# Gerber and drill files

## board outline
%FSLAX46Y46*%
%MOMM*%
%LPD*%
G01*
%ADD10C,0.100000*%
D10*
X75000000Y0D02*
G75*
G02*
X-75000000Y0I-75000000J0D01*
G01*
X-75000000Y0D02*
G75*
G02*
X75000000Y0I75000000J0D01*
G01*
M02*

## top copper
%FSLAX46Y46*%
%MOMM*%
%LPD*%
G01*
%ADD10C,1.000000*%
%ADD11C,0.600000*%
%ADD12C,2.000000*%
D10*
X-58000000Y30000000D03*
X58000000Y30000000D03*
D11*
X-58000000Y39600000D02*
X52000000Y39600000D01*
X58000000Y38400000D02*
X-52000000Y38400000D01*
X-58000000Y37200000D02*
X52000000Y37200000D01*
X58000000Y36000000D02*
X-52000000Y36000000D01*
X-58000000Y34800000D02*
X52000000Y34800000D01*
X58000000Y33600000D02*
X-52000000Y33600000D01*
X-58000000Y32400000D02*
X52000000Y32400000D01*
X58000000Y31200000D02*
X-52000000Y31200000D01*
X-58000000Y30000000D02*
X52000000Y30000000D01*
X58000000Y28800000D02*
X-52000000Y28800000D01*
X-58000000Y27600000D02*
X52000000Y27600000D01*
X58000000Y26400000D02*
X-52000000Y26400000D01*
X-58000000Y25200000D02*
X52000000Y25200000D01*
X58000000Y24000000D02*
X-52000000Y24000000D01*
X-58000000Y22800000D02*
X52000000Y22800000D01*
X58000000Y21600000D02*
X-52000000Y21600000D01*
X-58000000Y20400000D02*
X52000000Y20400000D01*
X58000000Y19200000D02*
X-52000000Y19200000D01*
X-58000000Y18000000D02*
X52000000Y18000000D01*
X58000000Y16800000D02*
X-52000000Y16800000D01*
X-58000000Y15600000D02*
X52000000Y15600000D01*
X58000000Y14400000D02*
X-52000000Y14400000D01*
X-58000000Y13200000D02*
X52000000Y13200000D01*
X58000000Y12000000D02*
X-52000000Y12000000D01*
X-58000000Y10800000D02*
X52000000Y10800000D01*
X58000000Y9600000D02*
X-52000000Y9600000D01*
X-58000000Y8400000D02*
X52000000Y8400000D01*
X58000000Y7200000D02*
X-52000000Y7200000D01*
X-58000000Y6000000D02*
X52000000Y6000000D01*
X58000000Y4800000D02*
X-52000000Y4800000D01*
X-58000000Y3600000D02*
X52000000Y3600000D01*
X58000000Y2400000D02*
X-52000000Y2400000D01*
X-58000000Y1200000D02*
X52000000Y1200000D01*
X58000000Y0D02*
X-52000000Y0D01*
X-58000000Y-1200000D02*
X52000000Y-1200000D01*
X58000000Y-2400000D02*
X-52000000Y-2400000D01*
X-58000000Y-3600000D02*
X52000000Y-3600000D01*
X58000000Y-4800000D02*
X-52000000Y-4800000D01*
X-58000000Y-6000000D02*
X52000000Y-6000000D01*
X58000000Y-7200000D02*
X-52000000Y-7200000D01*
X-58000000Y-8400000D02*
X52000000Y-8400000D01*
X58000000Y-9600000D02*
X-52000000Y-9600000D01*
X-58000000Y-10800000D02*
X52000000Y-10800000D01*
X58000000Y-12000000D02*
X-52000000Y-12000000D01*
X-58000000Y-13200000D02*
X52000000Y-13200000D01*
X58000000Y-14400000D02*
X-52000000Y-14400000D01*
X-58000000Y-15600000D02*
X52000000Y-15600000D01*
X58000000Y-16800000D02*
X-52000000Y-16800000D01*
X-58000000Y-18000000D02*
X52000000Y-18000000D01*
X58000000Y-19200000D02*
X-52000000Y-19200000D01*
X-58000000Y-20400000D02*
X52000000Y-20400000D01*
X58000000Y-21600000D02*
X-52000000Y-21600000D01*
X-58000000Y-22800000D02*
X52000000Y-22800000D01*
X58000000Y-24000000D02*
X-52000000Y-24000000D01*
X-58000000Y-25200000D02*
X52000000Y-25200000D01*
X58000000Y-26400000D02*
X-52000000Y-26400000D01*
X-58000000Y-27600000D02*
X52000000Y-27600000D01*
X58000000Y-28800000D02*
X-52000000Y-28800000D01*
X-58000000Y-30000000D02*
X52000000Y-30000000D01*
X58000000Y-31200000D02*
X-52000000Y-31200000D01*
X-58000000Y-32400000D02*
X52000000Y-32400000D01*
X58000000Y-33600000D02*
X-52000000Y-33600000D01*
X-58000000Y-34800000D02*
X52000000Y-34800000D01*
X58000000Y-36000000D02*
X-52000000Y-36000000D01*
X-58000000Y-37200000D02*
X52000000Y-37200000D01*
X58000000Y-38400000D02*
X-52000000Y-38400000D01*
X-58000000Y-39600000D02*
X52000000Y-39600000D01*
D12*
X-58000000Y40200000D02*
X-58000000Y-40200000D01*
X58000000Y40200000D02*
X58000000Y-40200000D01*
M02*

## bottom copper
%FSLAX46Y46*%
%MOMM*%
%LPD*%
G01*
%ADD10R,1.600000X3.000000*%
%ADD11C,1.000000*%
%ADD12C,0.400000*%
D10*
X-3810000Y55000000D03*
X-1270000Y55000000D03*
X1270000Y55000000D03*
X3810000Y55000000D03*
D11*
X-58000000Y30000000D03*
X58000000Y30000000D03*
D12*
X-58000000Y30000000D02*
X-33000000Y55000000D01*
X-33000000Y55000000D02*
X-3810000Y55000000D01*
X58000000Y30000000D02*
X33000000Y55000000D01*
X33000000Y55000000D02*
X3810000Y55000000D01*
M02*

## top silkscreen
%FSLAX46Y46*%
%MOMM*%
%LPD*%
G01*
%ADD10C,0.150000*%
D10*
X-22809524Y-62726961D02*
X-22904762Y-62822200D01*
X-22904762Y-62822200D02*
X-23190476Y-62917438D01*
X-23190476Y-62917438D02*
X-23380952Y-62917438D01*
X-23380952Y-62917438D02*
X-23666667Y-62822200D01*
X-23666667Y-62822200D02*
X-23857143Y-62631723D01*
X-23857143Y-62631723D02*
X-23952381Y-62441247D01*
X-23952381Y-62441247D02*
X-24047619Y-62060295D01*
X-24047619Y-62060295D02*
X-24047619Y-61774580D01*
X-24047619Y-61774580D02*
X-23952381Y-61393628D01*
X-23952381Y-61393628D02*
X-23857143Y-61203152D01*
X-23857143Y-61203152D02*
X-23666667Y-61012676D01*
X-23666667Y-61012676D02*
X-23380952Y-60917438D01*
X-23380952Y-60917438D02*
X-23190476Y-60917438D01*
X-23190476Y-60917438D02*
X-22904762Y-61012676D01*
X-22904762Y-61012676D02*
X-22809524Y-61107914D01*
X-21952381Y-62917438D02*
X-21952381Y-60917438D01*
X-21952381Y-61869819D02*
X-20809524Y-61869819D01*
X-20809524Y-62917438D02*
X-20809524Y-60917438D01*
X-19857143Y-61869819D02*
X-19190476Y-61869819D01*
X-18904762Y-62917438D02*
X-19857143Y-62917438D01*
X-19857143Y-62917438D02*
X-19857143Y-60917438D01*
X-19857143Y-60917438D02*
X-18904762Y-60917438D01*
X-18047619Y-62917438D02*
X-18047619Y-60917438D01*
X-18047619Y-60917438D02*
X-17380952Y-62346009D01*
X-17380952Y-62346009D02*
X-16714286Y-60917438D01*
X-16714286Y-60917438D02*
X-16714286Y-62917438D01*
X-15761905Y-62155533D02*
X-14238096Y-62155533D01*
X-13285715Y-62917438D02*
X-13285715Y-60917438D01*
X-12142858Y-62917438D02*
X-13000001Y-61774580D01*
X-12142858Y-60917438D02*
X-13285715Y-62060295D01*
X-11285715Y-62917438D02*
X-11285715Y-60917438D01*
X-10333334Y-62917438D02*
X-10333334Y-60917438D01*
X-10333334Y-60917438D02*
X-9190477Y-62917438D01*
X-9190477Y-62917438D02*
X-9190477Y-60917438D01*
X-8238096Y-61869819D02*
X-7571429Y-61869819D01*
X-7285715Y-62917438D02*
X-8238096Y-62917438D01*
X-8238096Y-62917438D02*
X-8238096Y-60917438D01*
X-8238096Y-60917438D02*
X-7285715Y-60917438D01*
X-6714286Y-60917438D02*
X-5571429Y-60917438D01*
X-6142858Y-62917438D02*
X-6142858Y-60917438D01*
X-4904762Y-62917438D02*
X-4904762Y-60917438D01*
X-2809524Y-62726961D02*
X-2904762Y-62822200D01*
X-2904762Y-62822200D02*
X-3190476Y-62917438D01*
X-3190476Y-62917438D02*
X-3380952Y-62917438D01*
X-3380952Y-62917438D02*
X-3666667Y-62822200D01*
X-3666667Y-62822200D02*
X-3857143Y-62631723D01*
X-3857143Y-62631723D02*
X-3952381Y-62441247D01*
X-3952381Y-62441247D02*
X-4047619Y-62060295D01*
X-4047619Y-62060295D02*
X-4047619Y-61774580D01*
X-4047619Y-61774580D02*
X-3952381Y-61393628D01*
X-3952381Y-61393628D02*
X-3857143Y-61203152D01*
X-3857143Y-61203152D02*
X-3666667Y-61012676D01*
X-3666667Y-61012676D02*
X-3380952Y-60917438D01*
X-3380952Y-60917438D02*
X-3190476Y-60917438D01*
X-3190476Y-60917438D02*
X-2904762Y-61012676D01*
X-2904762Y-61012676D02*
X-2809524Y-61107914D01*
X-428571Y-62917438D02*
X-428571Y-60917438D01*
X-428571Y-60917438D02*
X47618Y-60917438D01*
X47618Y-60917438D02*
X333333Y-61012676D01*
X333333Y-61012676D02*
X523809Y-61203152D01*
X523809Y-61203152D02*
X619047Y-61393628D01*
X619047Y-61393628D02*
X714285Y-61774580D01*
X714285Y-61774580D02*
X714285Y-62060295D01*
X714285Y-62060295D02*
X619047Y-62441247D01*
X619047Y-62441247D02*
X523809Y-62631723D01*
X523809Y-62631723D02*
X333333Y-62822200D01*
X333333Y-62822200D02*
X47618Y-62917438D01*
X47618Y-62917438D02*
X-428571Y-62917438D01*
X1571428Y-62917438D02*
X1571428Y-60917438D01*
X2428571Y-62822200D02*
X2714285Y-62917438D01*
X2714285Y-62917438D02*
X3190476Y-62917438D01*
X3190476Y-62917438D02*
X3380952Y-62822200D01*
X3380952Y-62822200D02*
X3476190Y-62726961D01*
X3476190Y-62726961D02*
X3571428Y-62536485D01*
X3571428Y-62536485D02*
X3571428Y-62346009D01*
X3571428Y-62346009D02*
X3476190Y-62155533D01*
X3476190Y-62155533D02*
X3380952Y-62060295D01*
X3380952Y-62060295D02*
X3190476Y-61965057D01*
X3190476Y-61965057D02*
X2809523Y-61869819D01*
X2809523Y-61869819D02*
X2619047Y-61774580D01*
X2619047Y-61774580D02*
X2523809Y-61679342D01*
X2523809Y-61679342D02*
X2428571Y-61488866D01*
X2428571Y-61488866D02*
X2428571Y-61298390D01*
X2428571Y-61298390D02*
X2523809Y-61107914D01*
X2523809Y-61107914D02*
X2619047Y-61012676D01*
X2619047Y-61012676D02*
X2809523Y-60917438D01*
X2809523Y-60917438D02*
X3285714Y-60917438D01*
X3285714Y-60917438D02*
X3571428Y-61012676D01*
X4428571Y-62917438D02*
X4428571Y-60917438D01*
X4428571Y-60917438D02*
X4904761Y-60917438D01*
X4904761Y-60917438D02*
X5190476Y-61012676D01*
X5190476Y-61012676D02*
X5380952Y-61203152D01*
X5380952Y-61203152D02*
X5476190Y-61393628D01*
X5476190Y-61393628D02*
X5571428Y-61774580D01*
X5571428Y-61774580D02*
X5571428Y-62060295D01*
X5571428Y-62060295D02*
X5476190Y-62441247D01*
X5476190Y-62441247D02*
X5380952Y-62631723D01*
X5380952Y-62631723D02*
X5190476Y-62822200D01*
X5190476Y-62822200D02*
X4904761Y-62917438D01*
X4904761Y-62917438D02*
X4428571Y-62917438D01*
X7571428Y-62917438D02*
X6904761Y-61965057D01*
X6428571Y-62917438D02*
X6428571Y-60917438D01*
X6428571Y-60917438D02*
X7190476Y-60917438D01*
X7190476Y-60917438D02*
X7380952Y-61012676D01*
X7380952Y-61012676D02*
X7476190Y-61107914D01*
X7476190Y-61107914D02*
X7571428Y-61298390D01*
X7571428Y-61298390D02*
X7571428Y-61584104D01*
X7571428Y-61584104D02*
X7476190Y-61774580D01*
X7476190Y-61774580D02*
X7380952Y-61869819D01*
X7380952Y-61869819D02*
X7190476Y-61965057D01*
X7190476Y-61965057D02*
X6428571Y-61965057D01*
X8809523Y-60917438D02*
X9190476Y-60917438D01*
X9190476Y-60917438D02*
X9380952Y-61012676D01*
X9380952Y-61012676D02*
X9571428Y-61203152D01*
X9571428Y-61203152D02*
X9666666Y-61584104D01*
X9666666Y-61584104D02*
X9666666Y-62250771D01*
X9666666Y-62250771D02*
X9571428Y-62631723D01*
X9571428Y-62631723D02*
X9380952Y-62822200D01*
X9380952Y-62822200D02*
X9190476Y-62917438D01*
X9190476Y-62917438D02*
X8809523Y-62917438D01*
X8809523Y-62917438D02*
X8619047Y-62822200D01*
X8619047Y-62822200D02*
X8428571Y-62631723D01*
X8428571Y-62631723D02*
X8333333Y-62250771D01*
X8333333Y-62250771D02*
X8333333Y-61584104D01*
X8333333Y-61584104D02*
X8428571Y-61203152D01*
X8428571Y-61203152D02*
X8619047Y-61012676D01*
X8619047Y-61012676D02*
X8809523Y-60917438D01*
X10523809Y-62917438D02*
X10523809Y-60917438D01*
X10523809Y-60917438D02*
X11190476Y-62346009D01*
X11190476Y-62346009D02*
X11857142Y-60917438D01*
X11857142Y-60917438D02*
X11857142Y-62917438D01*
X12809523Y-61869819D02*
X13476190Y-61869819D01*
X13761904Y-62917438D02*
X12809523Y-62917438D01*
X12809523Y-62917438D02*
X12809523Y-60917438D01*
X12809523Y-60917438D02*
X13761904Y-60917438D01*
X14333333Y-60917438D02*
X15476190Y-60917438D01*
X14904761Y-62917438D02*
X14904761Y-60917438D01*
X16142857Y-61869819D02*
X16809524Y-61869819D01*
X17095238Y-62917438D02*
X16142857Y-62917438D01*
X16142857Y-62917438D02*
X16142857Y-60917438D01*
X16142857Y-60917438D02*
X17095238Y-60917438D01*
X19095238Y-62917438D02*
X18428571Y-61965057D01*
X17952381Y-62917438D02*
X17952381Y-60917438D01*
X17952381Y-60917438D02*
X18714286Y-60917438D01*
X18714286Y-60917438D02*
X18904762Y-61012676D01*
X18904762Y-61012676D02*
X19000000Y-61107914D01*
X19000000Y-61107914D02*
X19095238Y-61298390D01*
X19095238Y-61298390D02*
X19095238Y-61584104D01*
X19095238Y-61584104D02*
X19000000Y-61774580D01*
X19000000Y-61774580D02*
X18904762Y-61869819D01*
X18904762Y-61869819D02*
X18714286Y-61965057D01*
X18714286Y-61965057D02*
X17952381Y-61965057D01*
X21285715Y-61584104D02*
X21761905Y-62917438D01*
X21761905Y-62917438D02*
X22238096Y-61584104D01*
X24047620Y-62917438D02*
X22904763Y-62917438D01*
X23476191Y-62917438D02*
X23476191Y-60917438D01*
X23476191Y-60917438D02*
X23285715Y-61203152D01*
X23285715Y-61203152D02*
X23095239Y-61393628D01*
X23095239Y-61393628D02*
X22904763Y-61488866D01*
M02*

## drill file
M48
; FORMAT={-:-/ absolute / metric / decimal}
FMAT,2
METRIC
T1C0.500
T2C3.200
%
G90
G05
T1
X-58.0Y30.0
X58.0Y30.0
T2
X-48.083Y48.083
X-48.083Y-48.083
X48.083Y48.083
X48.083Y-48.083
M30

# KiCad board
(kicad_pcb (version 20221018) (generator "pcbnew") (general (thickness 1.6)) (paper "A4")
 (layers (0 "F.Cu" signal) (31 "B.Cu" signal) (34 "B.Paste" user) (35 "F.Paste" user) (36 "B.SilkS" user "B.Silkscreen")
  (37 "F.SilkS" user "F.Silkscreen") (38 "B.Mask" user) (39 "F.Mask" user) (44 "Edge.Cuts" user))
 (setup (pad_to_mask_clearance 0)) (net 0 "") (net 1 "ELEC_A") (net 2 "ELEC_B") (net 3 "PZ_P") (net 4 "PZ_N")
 (segment (start -58.000 -39.600) (end 52.000 -39.600) (width 0.6) (layer "F.Cu") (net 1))
 (segment (start 58.000 -38.400) (end -52.000 -38.400) (width 0.6) (layer "F.Cu") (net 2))
 (segment (start -58.000 -37.200) (end 52.000 -37.200) (width 0.6) (layer "F.Cu") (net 1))
 (segment (start 58.000 -36.000) (end -52.000 -36.000) (width 0.6) (layer "F.Cu") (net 2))
 (segment (start -58.000 -34.800) (end 52.000 -34.800) (width 0.6) (layer "F.Cu") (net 1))
 (segment (start 58.000 -33.600) (end -52.000 -33.600) (width 0.6) (layer "F.Cu") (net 2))
 (segment (start -58.000 -32.400) (end 52.000 -32.400) (width 0.6) (layer "F.Cu") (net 1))
 (segment (start 58.000 -31.200) (end -52.000 -31.200) (width 0.6) (layer "F.Cu") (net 2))
 (segment (start -58.000 -30.000) (end 52.000 -30.000) (width 0.6) (layer "F.Cu") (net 1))
 (segment (start 58.000 -28.800) (end -52.000 -28.800) (width 0.6) (layer "F.Cu") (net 2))
 (segment (start -58.000 -27.600) (end 52.000 -27.600) (width 0.6) (layer "F.Cu") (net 1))
 (segment (start 58.000 -26.400) (end -52.000 -26.400) (width 0.6) (layer "F.Cu") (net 2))
 (segment (start -58.000 -25.200) (end 52.000 -25.200) (width 0.6) (layer "F.Cu") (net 1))
 (segment (start 58.000 -24.000) (end -52.000 -24.000) (width 0.6) (layer "F.Cu") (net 2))
 (segment (start -58.000 -22.800) (end 52.000 -22.800) (width 0.6) (layer "F.Cu") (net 1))
 (segment (start 58.000 -21.600) (end -52.000 -21.600) (width 0.6) (layer "F.Cu") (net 2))
 (segment (start -58.000 -20.400) (end 52.000 -20.400) (width 0.6) (layer "F.Cu") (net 1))
 (segment (start 58.000 -19.200) (end -52.000 -19.200) (width 0.6) (layer "F.Cu") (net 2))
 (segment (start -58.000 -18.000) (end 52.000 -18.000) (width 0.6) (layer "F.Cu") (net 1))
 (segment (start 58.000 -16.800) (end -52.000 -16.800) (width 0.6) (layer "F.Cu") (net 2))
 (segment (start -58.000 -15.600) (end 52.000 -15.600) (width 0.6) (layer "F.Cu") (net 1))
 (segment (start 58.000 -14.400) (end -52.000 -14.400) (width 0.6) (layer "F.Cu") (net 2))
 (segment (start -58.000 -13.200) (end 52.000 -13.200) (width 0.6) (layer "F.Cu") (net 1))
 (segment (start 58.000 -12.000) (end -52.000 -12.000) (width 0.6) (layer "F.Cu") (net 2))
 (segment (start -58.000 -10.800) (end 52.000 -10.800) (width 0.6) (layer "F.Cu") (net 1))
 (segment (start 58.000 -9.600) (end -52.000 -9.600) (width 0.6) (layer "F.Cu") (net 2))
 (segment (start -58.000 -8.400) (end 52.000 -8.400) (width 0.6) (layer "F.Cu") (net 1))
 (segment (start 58.000 -7.200) (end -52.000 -7.200) (width 0.6) (layer "F.Cu") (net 2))
 (segment (start -58.000 -6.000) (end 52.000 -6.000) (width 0.6) (layer "F.Cu") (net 1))
 (segment (start 58.000 -4.800) (end -52.000 -4.800) (width 0.6) (layer "F.Cu") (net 2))
 (segment (start -58.000 -3.600) (end 52.000 -3.600) (width 0.6) (layer "F.Cu") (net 1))
 (segment (start 58.000 -2.400) (end -52.000 -2.400) (width 0.6) (layer "F.Cu") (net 2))
 (segment (start -58.000 -1.200) (end 52.000 -1.200) (width 0.6) (layer "F.Cu") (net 1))
 (segment (start 58.000 0.000) (end -52.000 0.000) (width 0.6) (layer "F.Cu") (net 2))
 (segment (start -58.000 1.200) (end 52.000 1.200) (width 0.6) (layer "F.Cu") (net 1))
 (segment (start 58.000 2.400) (end -52.000 2.400) (width 0.6) (layer "F.Cu") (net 2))
 (segment (start -58.000 3.600) (end 52.000 3.600) (width 0.6) (layer "F.Cu") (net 1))
 (segment (start 58.000 4.800) (end -52.000 4.800) (width 0.6) (layer "F.Cu") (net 2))
 (segment (start -58.000 6.000) (end 52.000 6.000) (width 0.6) (layer "F.Cu") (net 1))
 (segment (start 58.000 7.200) (end -52.000 7.200) (width 0.6) (layer "F.Cu") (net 2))
 (segment (start -58.000 8.400) (end 52.000 8.400) (width 0.6) (layer "F.Cu") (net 1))
 (segment (start 58.000 9.600) (end -52.000 9.600) (width 0.6) (layer "F.Cu") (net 2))
 (segment (start -58.000 10.800) (end 52.000 10.800) (width 0.6) (layer "F.Cu") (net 1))
 (segment (start 58.000 12.000) (end -52.000 12.000) (width 0.6) (layer "F.Cu") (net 2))
 (segment (start -58.000 13.200) (end 52.000 13.200) (width 0.6) (layer "F.Cu") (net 1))
 (segment (start 58.000 14.400) (end -52.000 14.400) (width 0.6) (layer "F.Cu") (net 2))
 (segment (start -58.000 15.600) (end 52.000 15.600) (width 0.6) (layer "F.Cu") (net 1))
 (segment (start 58.000 16.800) (end -52.000 16.800) (width 0.6) (layer "F.Cu") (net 2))
 (segment (start -58.000 18.000) (end 52.000 18.000) (width 0.6) (layer "F.Cu") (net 1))
 (segment (start 58.000 19.200) (end -52.000 19.200) (width 0.6) (layer "F.Cu") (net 2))
 (segment (start -58.000 20.400) (end 52.000 20.400) (width 0.6) (layer "F.Cu") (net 1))
 (segment (start 58.000 21.600) (end -52.000 21.600) (width 0.6) (layer "F.Cu") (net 2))
 (segment (start -58.000 22.800) (end 52.000 22.800) (width 0.6) (layer "F.Cu") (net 1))
 (segment (start 58.000 24.000) (end -52.000 24.000) (width 0.6) (layer "F.Cu") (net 2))
 (segment (start -58.000 25.200) (end 52.000 25.200) (width 0.6) (layer "F.Cu") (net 1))
 (segment (start 58.000 26.400) (end -52.000 26.400) (width 0.6) (layer "F.Cu") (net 2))
 (segment (start -58.000 27.600) (end 52.000 27.600) (width 0.6) (layer "F.Cu") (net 1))
 (segment (start 58.000 28.800) (end -52.000 28.800) (width 0.6) (layer "F.Cu") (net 2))
 (segment (start -58.000 30.000) (end 52.000 30.000) (width 0.6) (layer "F.Cu") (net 1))
 (segment (start 58.000 31.200) (end -52.000 31.200) (width 0.6) (layer "F.Cu") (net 2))
 (segment (start -58.000 32.400) (end 52.000 32.400) (width 0.6) (layer "F.Cu") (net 1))
 (segment (start 58.000 33.600) (end -52.000 33.600) (width 0.6) (layer "F.Cu") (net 2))
 (segment (start -58.000 34.800) (end 52.000 34.800) (width 0.6) (layer "F.Cu") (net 1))
 (segment (start 58.000 36.000) (end -52.000 36.000) (width 0.6) (layer "F.Cu") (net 2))
 (segment (start -58.000 37.200) (end 52.000 37.200) (width 0.6) (layer "F.Cu") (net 1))
 (segment (start 58.000 38.400) (end -52.000 38.400) (width 0.6) (layer "F.Cu") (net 2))
 (segment (start -58.000 39.600) (end 52.000 39.600) (width 0.6) (layer "F.Cu") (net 1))
 (segment (start -58.000 -40.200) (end -58.000 40.200) (width 2.0) (layer "F.Cu") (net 1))
 (segment (start 58.000 -40.200) (end 58.000 40.200) (width 2.0) (layer "F.Cu") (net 2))
 (via (at -58.0 -30) (size 1.0) (drill 0.5) (layers "F.Cu" "B.Cu") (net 1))
 (segment (start -58.000 -30.000) (end -33.000 -55.000) (width 0.4) (layer "B.Cu") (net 1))
 (segment (start -33.000 -55.000) (end -3.810 -55.000) (width 0.4) (layer "B.Cu") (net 1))
 (via (at 58.0 -30) (size 1.0) (drill 0.5) (layers "F.Cu" "B.Cu") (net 2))
 (segment (start 58.000 -30.000) (end 33.000 -55.000) (width 0.4) (layer "B.Cu") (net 2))
 (segment (start 33.000 -55.000) (end 3.810 -55.000) (width 0.4) (layer "B.Cu") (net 2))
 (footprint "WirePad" (layer "F.Cu") (at -3.81 -55) (pad "1" smd rect (at 0 0) (size 1.6 3.0) (layers "B.Cu" "B.Mask") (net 1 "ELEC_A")))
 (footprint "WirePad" (layer "F.Cu") (at -1.27 -55) (pad "1" smd rect (at 0 0) (size 1.6 3.0) (layers "B.Cu" "B.Mask") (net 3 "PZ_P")))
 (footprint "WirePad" (layer "F.Cu") (at 1.27 -55) (pad "1" smd rect (at 0 0) (size 1.6 3.0) (layers "B.Cu" "B.Mask") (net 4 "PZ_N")))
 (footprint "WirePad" (layer "F.Cu") (at 3.81 -55) (pad "1" smd rect (at 0 0) (size 1.6 3.0) (layers "B.Cu" "B.Mask") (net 2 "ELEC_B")))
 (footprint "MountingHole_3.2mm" (layer "F.Cu") (at 48.083 48.083)
  (pad "" np_thru_hole circle (at 0 0) (size 3.2 3.2) (drill 3.2) (layers "*.Cu" "*.Mask")))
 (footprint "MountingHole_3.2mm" (layer "F.Cu") (at -48.083 48.083)
  (pad "" np_thru_hole circle (at 0 0) (size 3.2 3.2) (drill 3.2) (layers "*.Cu" "*.Mask")))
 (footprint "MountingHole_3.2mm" (layer "F.Cu") (at -48.083 -48.083)
  (pad "" np_thru_hole circle (at 0 0) (size 3.2 3.2) (drill 3.2) (layers "*.Cu" "*.Mask")))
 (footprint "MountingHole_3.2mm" (layer "F.Cu") (at 48.083 -48.083)
  (pad "" np_thru_hole circle (at 0 0) (size 3.2 3.2) (drill 3.2) (layers "*.Cu" "*.Mask")))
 (gr_circle (center 0 0) (end 75.0 0) (stroke (width 0.1) (type default)) (fill none) (layer "Edge.Cuts"))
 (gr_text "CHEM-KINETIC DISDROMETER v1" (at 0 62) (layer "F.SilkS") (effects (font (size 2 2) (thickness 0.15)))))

